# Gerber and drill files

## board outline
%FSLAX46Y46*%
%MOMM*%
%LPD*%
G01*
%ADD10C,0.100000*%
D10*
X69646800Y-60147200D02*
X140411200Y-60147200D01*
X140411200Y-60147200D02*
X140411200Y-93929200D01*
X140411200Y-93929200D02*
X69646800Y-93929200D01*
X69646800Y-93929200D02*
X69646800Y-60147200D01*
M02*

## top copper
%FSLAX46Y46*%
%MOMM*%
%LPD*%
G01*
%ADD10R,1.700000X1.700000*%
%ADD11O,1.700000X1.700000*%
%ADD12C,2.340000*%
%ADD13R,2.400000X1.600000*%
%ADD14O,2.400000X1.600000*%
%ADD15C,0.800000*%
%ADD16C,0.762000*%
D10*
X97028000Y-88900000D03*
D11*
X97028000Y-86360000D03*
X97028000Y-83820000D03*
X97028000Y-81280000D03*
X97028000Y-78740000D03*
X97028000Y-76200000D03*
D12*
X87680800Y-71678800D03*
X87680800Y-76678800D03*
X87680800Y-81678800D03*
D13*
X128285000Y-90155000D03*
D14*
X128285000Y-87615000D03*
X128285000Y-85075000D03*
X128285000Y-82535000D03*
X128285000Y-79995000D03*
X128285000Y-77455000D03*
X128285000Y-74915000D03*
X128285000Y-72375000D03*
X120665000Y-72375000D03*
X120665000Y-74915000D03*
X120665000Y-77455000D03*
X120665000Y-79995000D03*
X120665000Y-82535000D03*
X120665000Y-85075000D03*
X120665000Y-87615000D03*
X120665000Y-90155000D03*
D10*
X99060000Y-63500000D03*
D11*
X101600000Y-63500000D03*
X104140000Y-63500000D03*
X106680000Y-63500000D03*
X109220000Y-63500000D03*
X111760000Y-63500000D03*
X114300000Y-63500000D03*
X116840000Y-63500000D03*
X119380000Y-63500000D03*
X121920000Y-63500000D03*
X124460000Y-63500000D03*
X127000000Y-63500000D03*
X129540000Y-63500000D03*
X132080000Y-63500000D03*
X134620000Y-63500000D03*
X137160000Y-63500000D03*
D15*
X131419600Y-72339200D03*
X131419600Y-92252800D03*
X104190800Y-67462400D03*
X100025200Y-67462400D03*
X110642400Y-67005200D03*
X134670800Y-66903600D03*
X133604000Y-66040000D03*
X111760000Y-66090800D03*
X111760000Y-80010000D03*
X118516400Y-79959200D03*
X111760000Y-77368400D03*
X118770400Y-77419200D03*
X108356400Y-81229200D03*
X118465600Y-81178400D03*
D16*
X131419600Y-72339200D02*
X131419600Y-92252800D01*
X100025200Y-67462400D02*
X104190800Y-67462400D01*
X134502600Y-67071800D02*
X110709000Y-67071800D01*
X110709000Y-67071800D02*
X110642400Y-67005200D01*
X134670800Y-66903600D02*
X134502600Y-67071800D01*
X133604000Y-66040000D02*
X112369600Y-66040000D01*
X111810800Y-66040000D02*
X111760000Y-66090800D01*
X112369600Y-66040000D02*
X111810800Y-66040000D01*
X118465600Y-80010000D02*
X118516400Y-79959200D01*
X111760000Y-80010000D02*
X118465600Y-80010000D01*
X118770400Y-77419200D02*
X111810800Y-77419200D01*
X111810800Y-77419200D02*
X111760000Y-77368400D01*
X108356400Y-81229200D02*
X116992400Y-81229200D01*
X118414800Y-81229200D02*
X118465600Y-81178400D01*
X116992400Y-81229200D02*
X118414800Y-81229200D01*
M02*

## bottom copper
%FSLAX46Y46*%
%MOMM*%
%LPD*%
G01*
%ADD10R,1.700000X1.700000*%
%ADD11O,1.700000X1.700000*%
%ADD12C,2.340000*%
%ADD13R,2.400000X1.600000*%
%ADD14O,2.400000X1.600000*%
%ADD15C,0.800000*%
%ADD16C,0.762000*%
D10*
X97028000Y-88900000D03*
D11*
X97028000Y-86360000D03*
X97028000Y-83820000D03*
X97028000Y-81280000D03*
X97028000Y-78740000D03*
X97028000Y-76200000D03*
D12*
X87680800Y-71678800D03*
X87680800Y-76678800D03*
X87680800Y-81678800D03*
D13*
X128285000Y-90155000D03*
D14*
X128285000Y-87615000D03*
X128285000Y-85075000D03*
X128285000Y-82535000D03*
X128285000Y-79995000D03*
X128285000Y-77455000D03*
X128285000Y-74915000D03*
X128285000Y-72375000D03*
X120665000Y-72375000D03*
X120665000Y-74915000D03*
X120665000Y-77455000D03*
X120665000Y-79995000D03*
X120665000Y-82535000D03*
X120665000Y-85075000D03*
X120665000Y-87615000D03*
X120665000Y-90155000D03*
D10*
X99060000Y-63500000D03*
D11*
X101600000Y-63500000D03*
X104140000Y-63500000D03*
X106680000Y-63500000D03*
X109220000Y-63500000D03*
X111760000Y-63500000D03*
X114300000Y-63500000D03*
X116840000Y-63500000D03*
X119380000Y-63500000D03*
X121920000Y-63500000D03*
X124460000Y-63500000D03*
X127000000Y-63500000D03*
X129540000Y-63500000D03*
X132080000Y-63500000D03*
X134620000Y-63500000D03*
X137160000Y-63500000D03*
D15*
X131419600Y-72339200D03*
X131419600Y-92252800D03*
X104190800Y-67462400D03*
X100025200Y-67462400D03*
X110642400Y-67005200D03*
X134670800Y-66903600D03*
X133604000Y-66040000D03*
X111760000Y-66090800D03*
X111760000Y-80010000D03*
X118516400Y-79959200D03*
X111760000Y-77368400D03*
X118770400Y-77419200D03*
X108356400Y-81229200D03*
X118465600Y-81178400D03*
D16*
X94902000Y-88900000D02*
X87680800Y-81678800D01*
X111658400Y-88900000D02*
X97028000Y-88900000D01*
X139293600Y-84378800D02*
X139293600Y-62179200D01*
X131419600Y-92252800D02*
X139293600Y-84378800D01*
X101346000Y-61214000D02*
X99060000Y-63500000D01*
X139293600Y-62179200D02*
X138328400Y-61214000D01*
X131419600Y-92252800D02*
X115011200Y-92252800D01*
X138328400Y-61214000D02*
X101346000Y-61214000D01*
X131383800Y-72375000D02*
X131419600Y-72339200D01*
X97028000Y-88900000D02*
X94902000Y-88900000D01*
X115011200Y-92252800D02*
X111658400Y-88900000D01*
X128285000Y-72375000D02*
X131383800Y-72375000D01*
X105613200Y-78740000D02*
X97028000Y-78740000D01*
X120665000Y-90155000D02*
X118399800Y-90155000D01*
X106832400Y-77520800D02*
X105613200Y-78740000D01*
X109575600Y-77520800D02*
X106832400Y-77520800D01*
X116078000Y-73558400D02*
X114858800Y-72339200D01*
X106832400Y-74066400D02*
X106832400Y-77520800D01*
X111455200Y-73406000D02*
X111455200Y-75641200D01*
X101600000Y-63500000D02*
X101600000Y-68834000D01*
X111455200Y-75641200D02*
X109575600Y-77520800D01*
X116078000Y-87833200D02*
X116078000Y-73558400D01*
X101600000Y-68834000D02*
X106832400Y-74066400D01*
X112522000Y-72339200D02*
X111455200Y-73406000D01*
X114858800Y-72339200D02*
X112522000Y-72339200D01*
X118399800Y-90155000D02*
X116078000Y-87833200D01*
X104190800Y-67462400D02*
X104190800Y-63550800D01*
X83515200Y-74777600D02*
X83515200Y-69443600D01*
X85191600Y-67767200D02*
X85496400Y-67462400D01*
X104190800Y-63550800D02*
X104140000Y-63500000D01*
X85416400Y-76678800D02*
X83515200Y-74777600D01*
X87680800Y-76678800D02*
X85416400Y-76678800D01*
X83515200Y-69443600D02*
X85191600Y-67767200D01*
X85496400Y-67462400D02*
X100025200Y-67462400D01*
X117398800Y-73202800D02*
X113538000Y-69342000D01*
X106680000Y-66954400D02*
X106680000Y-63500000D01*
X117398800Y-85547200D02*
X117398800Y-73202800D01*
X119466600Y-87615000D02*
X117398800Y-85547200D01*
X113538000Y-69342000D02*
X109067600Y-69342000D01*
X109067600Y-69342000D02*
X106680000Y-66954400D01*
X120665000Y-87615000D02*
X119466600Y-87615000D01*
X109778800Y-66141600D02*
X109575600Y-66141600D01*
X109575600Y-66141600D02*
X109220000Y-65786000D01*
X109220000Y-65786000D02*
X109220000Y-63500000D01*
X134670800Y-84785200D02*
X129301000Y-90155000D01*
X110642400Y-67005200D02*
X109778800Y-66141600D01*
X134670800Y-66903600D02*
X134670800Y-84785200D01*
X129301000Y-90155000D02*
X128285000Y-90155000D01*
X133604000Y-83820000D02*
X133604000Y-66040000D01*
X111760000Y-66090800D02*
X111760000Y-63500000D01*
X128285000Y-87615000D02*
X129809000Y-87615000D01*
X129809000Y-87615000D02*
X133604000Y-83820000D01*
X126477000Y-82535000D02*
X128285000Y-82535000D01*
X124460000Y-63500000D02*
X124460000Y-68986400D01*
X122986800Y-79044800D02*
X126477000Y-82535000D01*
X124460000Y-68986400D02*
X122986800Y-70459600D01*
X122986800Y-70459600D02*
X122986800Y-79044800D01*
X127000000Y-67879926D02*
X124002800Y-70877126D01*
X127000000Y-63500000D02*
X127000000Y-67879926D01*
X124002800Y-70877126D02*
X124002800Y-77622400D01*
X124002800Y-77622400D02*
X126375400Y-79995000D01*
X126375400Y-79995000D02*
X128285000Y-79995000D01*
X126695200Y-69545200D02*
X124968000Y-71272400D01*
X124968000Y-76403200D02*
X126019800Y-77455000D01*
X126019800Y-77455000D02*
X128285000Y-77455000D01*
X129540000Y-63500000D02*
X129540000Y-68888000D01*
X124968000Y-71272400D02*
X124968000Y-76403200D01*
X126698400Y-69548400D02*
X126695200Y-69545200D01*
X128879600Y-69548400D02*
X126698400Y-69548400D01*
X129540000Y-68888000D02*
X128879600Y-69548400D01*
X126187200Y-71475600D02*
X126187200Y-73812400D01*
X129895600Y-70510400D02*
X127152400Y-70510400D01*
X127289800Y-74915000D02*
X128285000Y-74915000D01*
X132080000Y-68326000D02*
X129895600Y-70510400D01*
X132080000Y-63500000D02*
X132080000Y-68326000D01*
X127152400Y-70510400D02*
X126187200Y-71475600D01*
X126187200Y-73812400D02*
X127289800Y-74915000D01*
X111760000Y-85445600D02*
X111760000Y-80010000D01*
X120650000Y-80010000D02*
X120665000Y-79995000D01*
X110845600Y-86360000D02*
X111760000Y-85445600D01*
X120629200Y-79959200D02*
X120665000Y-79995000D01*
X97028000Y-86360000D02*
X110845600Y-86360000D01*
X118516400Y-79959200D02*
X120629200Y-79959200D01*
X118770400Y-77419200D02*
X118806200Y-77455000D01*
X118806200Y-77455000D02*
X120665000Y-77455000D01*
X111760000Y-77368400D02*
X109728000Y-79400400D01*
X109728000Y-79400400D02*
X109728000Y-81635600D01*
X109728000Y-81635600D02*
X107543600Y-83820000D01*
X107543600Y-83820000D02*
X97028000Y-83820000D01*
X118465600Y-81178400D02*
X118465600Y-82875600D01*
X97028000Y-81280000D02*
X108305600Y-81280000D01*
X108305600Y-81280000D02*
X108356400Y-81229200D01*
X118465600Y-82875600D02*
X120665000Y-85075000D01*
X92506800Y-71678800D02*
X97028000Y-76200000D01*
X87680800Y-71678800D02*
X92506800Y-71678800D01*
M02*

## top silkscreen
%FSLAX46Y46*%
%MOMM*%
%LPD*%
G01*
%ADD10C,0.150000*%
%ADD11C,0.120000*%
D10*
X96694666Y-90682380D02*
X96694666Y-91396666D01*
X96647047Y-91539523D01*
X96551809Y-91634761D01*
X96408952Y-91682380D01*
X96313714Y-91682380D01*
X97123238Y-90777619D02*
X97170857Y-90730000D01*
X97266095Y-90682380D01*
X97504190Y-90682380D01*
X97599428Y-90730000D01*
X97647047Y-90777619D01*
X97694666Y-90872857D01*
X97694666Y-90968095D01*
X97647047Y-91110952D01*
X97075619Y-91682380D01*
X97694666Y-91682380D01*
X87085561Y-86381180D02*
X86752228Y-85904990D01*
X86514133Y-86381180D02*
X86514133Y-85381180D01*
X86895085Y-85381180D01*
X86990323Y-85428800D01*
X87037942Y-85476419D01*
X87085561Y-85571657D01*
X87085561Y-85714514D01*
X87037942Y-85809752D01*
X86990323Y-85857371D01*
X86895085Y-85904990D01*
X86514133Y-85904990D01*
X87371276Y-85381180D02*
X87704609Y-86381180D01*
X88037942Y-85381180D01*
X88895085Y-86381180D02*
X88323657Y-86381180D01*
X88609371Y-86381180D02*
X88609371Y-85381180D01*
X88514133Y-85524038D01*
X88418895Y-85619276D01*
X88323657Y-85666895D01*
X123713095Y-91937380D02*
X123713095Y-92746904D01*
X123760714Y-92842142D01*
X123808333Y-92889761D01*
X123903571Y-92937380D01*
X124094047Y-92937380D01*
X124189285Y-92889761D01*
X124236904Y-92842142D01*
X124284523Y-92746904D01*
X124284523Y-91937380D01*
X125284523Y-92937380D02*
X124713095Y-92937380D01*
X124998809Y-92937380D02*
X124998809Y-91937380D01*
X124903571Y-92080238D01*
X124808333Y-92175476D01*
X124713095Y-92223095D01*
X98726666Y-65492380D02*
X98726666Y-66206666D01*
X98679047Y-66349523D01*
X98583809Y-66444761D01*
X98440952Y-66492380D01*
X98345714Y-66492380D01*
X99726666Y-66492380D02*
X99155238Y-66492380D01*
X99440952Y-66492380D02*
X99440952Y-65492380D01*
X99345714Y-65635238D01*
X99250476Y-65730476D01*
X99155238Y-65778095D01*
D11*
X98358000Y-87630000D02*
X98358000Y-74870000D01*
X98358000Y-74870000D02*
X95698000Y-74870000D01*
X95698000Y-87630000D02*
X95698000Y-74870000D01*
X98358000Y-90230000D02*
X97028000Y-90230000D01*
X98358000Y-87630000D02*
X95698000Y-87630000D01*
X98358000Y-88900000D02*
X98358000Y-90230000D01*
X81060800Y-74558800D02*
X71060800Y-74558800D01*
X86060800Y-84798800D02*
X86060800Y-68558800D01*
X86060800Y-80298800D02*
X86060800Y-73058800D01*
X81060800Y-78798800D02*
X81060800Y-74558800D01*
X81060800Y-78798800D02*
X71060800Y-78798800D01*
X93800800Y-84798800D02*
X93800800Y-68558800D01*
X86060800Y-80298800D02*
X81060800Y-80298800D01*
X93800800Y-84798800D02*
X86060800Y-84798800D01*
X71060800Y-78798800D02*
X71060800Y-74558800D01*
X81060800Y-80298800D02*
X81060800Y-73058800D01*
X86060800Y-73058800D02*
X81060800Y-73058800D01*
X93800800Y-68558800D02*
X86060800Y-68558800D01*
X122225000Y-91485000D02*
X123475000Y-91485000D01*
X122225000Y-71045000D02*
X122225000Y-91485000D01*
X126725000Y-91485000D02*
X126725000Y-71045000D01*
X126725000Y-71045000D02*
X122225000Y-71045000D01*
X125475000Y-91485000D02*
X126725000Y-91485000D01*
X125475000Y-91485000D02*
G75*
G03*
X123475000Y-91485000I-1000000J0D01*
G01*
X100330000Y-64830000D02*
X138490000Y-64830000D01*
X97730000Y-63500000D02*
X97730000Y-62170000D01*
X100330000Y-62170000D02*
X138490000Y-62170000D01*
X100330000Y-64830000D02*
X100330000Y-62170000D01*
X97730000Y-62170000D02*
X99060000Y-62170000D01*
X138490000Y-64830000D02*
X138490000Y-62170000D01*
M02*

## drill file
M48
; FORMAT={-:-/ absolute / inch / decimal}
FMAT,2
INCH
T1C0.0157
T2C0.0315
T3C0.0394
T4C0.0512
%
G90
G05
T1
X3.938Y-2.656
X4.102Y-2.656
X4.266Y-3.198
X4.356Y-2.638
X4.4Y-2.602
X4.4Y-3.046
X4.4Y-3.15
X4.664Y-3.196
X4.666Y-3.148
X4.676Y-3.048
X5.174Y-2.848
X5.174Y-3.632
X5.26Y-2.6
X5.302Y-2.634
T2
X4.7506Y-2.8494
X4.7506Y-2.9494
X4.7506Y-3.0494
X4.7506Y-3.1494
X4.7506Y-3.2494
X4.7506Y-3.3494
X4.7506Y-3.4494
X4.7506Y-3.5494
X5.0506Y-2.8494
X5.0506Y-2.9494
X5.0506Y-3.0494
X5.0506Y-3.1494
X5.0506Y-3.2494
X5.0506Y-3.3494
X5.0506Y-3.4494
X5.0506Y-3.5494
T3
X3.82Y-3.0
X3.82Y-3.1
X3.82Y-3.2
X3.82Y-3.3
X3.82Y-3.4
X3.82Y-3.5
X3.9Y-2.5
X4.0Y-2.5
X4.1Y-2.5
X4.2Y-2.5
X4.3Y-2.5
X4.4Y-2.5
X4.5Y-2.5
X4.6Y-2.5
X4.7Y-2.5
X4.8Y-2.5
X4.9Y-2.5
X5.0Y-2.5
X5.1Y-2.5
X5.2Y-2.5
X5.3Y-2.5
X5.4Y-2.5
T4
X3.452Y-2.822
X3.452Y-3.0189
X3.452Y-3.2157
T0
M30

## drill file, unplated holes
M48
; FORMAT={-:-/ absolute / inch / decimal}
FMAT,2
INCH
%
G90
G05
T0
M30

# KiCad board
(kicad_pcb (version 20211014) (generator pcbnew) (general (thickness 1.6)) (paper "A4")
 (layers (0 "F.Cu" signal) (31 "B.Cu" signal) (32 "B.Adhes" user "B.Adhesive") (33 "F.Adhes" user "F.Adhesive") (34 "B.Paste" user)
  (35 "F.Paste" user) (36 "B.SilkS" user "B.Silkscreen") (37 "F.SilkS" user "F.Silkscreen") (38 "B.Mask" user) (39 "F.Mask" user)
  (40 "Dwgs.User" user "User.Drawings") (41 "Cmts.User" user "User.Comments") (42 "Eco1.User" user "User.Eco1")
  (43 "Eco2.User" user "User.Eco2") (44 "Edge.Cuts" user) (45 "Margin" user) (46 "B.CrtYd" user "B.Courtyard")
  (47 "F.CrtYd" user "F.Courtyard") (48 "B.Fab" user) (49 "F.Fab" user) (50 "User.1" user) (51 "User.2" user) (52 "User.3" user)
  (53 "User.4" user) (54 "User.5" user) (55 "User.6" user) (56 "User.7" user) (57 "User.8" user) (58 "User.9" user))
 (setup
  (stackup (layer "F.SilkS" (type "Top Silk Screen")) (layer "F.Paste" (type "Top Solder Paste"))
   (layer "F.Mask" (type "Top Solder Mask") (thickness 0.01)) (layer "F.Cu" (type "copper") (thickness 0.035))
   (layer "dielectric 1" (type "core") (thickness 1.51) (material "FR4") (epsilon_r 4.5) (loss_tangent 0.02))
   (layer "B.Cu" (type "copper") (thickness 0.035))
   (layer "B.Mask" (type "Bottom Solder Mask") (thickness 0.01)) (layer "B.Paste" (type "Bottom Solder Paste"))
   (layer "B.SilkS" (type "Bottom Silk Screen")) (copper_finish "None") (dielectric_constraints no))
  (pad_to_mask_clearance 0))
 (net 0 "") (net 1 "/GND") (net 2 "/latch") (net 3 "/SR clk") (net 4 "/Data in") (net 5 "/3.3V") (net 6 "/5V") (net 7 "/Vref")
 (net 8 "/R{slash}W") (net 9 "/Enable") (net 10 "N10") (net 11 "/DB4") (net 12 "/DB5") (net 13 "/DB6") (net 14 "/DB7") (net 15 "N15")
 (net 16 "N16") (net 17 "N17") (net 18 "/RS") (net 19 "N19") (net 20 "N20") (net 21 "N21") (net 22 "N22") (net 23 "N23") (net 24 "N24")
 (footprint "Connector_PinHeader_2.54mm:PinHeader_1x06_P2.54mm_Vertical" (layer "F.Cu") (at 97.028 88.9 180)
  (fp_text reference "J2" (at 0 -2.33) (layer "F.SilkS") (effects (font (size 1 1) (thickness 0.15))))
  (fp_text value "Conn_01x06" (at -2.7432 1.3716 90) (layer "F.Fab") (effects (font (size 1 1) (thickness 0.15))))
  (fp_line (start -1.33 1.27) (end -1.33 14.03) (layer "F.SilkS") (width 0.12))
  (fp_line (start -1.33 14.03) (end 1.33 14.03) (layer "F.SilkS") (width 0.12))
  (fp_line (start 1.33 1.27) (end 1.33 14.03) (layer "F.SilkS") (width 0.12))
  (fp_line (start -1.33 -1.33) (end 0 -1.33) (layer "F.SilkS") (width 0.12))
  (fp_line (start -1.33 1.27) (end 1.33 1.27) (layer "F.SilkS") (width 0.12))
  (fp_line (start -1.33 0) (end -1.33 -1.33) (layer "F.SilkS") (width 0.12))
  (pad "1" thru_hole rect (at 0 0 180) (size 1.7 1.7) (drill 1) (layers *.Cu *.Mask) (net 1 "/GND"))
  (pad "2" thru_hole oval (at 0 2.54 180) (size 1.7 1.7) (drill 1) (layers *.Cu *.Mask) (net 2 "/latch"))
  (pad "3" thru_hole oval (at 0 5.08 180) (size 1.7 1.7) (drill 1) (layers *.Cu *.Mask) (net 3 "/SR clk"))
  (pad "4" thru_hole oval (at 0 7.62 180) (size 1.7 1.7) (drill 1) (layers *.Cu *.Mask) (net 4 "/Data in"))
  (pad "5" thru_hole oval (at 0 10.16 180) (size 1.7 1.7) (drill 1) (layers *.Cu *.Mask) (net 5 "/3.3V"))
  (pad "6" thru_hole oval (at 0 12.7 180) (size 1.7 1.7) (drill 1) (layers *.Cu *.Mask) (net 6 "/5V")))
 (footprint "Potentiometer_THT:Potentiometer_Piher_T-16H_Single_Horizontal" (layer "F.Cu") (at 87.6808 71.6788 180)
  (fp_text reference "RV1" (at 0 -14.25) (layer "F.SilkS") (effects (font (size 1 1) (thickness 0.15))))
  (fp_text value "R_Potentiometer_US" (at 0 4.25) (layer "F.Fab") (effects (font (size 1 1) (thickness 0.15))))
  (fp_line (start 6.62 -2.88) (end 16.62 -2.88) (layer "F.SilkS") (width 0.12))
  (fp_line (start 1.62 -13.12) (end 1.62 3.12) (layer "F.SilkS") (width 0.12))
  (fp_line (start 1.62 -8.62) (end 1.62 -1.38) (layer "F.SilkS") (width 0.12))
  (fp_line (start 6.62 -7.12) (end 6.62 -2.88) (layer "F.SilkS") (width 0.12))
  (fp_line (start 6.62 -7.12) (end 16.62 -7.12) (layer "F.SilkS") (width 0.12))
  (fp_line (start -6.12 -13.12) (end -6.12 3.12) (layer "F.SilkS") (width 0.12))
  (fp_line (start 1.62 -8.62) (end 6.62 -8.62) (layer "F.SilkS") (width 0.12))
  (fp_line (start -6.12 -13.12) (end 1.62 -13.12) (layer "F.SilkS") (width 0.12))
  (fp_line (start 16.62 -7.12) (end 16.62 -2.88) (layer "F.SilkS") (width 0.12))
  (fp_line (start 6.62 -8.62) (end 6.62 -1.38) (layer "F.SilkS") (width 0.12))
  (fp_line (start 1.62 -1.38) (end 6.62 -1.38) (layer "F.SilkS") (width 0.12))
  (fp_line (start -6.12 3.12) (end 1.62 3.12) (layer "F.SilkS") (width 0.12))
  (pad "1" thru_hole circle (at 0 0 180) (size 2.34 2.34) (drill 1.3) (layers *.Cu *.Mask) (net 6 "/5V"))
  (pad "2" thru_hole circle (at 0 -5 180) (size 2.34 2.34) (drill 1.3) (layers *.Cu *.Mask) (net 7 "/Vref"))
  (pad "3" thru_hole circle (at 0 -10 180) (size 2.34 2.34) (drill 1.3) (layers *.Cu *.Mask) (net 1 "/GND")))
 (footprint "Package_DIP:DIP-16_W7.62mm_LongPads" (layer "F.Cu") (at 128.285 90.155 180)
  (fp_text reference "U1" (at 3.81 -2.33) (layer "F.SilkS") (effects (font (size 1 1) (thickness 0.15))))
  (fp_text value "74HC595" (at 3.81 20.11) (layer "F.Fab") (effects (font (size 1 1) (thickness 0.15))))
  (fp_line (start 6.06 -1.33) (end 4.81 -1.33) (layer "F.SilkS") (width 0.12))
  (fp_line (start 6.06 19.11) (end 6.06 -1.33) (layer "F.SilkS") (width 0.12))
  (fp_line (start 1.56 -1.33) (end 1.56 19.11) (layer "F.SilkS") (width 0.12))
  (fp_line (start 1.56 19.11) (end 6.06 19.11) (layer "F.SilkS") (width 0.12))
  (fp_line (start 2.81 -1.33) (end 1.56 -1.33) (layer "F.SilkS") (width 0.12))
  (fp_arc (start 4.81 -1.33) (mid 3.81 -0.33) (end 2.81 -1.33) (layer "F.SilkS") (width 0.12))
  (pad "1" thru_hole rect (at 0 0 180) (size 2.4 1.6) (drill 0.8) (layers *.Cu *.Mask) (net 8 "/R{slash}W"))
  (pad "2" thru_hole oval (at 0 2.54 180) (size 2.4 1.6) (drill 0.8) (layers *.Cu *.Mask) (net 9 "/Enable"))
  (pad "3" thru_hole oval (at 0 5.08 180) (size 2.4 1.6) (drill 0.8) (layers *.Cu *.Mask) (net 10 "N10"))
  (pad "4" thru_hole oval (at 0 7.62 180) (size 2.4 1.6) (drill 0.8) (layers *.Cu *.Mask) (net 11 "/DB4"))
  (pad "5" thru_hole oval (at 0 10.16 180) (size 2.4 1.6) (drill 0.8) (layers *.Cu *.Mask) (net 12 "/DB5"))
  (pad "6" thru_hole oval (at 0 12.7 180) (size 2.4 1.6) (drill 0.8) (layers *.Cu *.Mask) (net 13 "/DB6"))
  (pad "7" thru_hole oval (at 0 15.24 180) (size 2.4 1.6) (drill 0.8) (layers *.Cu *.Mask) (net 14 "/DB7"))
  (pad "8" thru_hole oval (at 0 17.78 180) (size 2.4 1.6) (drill 0.8) (layers *.Cu *.Mask) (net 1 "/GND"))
  (pad "9" thru_hole oval (at 7.62 17.78 180) (size 2.4 1.6) (drill 0.8) (layers *.Cu *.Mask) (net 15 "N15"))
  (pad "10" thru_hole oval (at 7.62 15.24 180) (size 2.4 1.6) (drill 0.8) (layers *.Cu *.Mask) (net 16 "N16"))
  (pad "11" thru_hole oval (at 7.62 12.7 180) (size 2.4 1.6) (drill 0.8) (layers *.Cu *.Mask) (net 3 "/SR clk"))
  (pad "12" thru_hole oval (at 7.62 10.16 180) (size 2.4 1.6) (drill 0.8) (layers *.Cu *.Mask) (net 2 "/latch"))
  (pad "13" thru_hole oval (at 7.62 7.62 180) (size 2.4 1.6) (drill 0.8) (layers *.Cu *.Mask) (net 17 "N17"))
  (pad "14" thru_hole oval (at 7.62 5.08 180) (size 2.4 1.6) (drill 0.8) (layers *.Cu *.Mask) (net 4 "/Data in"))
  (pad "15" thru_hole oval (at 7.62 2.54 180) (size 2.4 1.6) (drill 0.8) (layers *.Cu *.Mask) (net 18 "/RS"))
  (pad "16" thru_hole oval (at 7.62 0 180) (size 2.4 1.6) (drill 0.8) (layers *.Cu *.Mask) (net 5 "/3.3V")))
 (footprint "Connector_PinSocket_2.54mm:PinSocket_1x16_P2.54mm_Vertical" (layer "F.Cu") (at 99.06 63.5 90)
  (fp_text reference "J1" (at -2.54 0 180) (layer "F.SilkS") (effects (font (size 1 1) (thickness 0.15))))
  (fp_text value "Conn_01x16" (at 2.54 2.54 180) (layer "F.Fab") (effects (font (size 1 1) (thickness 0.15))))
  (fp_line (start -1.33 1.27) (end -1.33 39.43) (layer "F.SilkS") (width 0.12))
  (fp_line (start 0 -1.33) (end 1.33 -1.33) (layer "F.SilkS") (width 0.12))
  (fp_line (start 1.33 1.27) (end 1.33 39.43) (layer "F.SilkS") (width 0.12))
  (fp_line (start -1.33 1.27) (end 1.33 1.27) (layer "F.SilkS") (width 0.12))
  (fp_line (start 1.33 -1.33) (end 1.33 0) (layer "F.SilkS") (width 0.12))
  (fp_line (start -1.33 39.43) (end 1.33 39.43) (layer "F.SilkS") (width 0.12))
  (pad "1" thru_hole rect (at 0 0 90) (size 1.7 1.7) (drill 1) (layers *.Cu *.Mask) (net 1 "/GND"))
  (pad "2" thru_hole oval (at 0 2.54 90) (size 1.7 1.7) (drill 1) (layers *.Cu *.Mask) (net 5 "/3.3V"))
  (pad "3" thru_hole oval (at 0 5.08 90) (size 1.7 1.7) (drill 1) (layers *.Cu *.Mask) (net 7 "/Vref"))
  (pad "4" thru_hole oval (at 0 7.62 90) (size 1.7 1.7) (drill 1) (layers *.Cu *.Mask) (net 18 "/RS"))
  (pad "5" thru_hole oval (at 0 10.16 90) (size 1.7 1.7) (drill 1) (layers *.Cu *.Mask) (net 8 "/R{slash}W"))
  (pad "6" thru_hole oval (at 0 12.7 90) (size 1.7 1.7) (drill 1) (layers *.Cu *.Mask) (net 9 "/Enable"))
  (pad "7" thru_hole oval (at 0 15.24 90) (size 1.7 1.7) (drill 1) (layers *.Cu *.Mask) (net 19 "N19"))
  (pad "8" thru_hole oval (at 0 17.78 90) (size 1.7 1.7) (drill 1) (layers *.Cu *.Mask) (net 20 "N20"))
  (pad "9" thru_hole oval (at 0 20.32 90) (size 1.7 1.7) (drill 1) (layers *.Cu *.Mask) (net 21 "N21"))
  (pad "10" thru_hole oval (at 0 22.86 90) (size 1.7 1.7) (drill 1) (layers *.Cu *.Mask) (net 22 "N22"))
  (pad "11" thru_hole oval (at 0 25.4 90) (size 1.7 1.7) (drill 1) (layers *.Cu *.Mask) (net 11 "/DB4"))
  (pad "12" thru_hole oval (at 0 27.94 90) (size 1.7 1.7) (drill 1) (layers *.Cu *.Mask) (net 12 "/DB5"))
  (pad "13" thru_hole oval (at 0 30.48 90) (size 1.7 1.7) (drill 1) (layers *.Cu *.Mask) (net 13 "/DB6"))
  (pad "14" thru_hole oval (at 0 33.02 90) (size 1.7 1.7) (drill 1) (layers *.Cu *.Mask) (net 14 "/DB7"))
  (pad "15" thru_hole oval (at 0 35.56 90) (size 1.7 1.7) (drill 1) (layers *.Cu *.Mask) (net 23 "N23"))
  (pad "16" thru_hole oval (at 0 38.1 90) (size 1.7 1.7) (drill 1) (layers *.Cu *.Mask) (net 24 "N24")))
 (gr_rect (start 69.6468 60.1472) (end 140.4112 93.9292) (layer "Edge.Cuts") (width 0.1) (fill none))
 (segment (start 131.4196 72.3392) (end 131.4196 92.2528) (width 0.762) (layer "F.Cu") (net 1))
 (via (at 131.4196 72.3392) (size 0.8) (drill 0.4) (layers "F.Cu" "B.Cu") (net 1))
 (via (at 131.4196 92.2528) (size 0.8) (drill 0.4) (layers "F.Cu" "B.Cu") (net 1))
 (segment (start 94.902 88.9) (end 87.6808 81.6788) (width 0.762) (layer "B.Cu") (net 1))
 (segment (start 111.6584 88.9) (end 97.028 88.9) (width 0.762) (layer "B.Cu") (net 1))
 (segment (start 139.2936 84.3788) (end 139.2936 62.1792) (width 0.762) (layer "B.Cu") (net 1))
 (segment (start 131.4196 92.2528) (end 139.2936 84.3788) (width 0.762) (layer "B.Cu") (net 1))
 (segment (start 101.346 61.214) (end 99.06 63.5) (width 0.762) (layer "B.Cu") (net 1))
 (segment (start 139.2936 62.1792) (end 138.3284 61.214) (width 0.762) (layer "B.Cu") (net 1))
 (segment (start 131.4196 92.2528) (end 115.0112 92.2528) (width 0.762) (layer "B.Cu") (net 1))
 (segment (start 138.3284 61.214) (end 101.346 61.214) (width 0.762) (layer "B.Cu") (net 1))
 (segment (start 131.3838 72.375) (end 131.4196 72.3392) (width 0.762) (layer "B.Cu") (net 1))
 (segment (start 97.028 88.9) (end 94.902 88.9) (width 0.762) (layer "B.Cu") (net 1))
 (segment (start 115.0112 92.2528) (end 111.6584 88.9) (width 0.762) (layer "B.Cu") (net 1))
 (segment (start 128.285 72.375) (end 131.3838 72.375) (width 0.762) (layer "B.Cu") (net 1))
 (segment (start 105.6132 78.74) (end 97.028 78.74) (width 0.762) (layer "B.Cu") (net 5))
 (segment (start 120.665 90.155) (end 118.3998 90.155) (width 0.762) (layer "B.Cu") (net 5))
 (segment (start 106.8324 77.5208) (end 105.6132 78.74) (width 0.762) (layer "B.Cu") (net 5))
 (segment (start 109.5756 77.5208) (end 106.8324 77.5208) (width 0.762) (layer "B.Cu") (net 5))
 (segment (start 116.078 73.5584) (end 114.8588 72.3392) (width 0.762) (layer "B.Cu") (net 5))
 (segment (start 106.8324 74.0664) (end 106.8324 77.5208) (width 0.762) (layer "B.Cu") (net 5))
 (segment (start 111.4552 73.406) (end 111.4552 75.6412) (width 0.762) (layer "B.Cu") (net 5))
 (segment (start 101.6 63.5) (end 101.6 68.834) (width 0.762) (layer "B.Cu") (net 5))
 (segment (start 111.4552 75.6412) (end 109.5756 77.5208) (width 0.762) (layer "B.Cu") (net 5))
 (segment (start 116.078 87.8332) (end 116.078 73.5584) (width 0.762) (layer "B.Cu") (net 5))
 (segment (start 101.6 68.834) (end 106.8324 74.0664) (width 0.762) (layer "B.Cu") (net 5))
 (segment (start 112.522 72.3392) (end 111.4552 73.406) (width 0.762) (layer "B.Cu") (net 5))
 (segment (start 114.8588 72.3392) (end 112.522 72.3392) (width 0.762) (layer "B.Cu") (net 5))
 (segment (start 118.3998 90.155) (end 116.078 87.8332) (width 0.762) (layer "B.Cu") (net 5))
 (segment (start 100.0252 67.4624) (end 104.1908 67.4624) (width 0.762) (layer "F.Cu") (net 7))
 (via (at 104.1908 67.4624) (size 0.8) (drill 0.4) (layers "F.Cu" "B.Cu") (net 7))
 (via (at 100.0252 67.4624) (size 0.8) (drill 0.4) (layers "F.Cu" "B.Cu") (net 7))
 (segment (start 104.1908 67.4624) (end 104.1908 63.5508) (width 0.762) (layer "B.Cu") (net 7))
 (segment (start 83.5152 74.7776) (end 83.5152 69.4436) (width 0.762) (layer "B.Cu") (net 7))
 (segment (start 85.1916 67.7672) (end 85.4964 67.4624) (width 0.762) (layer "B.Cu") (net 7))
 (segment (start 104.1908 63.5508) (end 104.14 63.5) (width 0.762) (layer "B.Cu") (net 7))
 (segment (start 85.4164 76.6788) (end 83.5152 74.7776) (width 0.762) (layer "B.Cu") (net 7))
 (segment (start 87.6808 76.6788) (end 85.4164 76.6788) (width 0.762) (layer "B.Cu") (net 7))
 (segment (start 83.5152 69.4436) (end 85.1916 67.7672) (width 0.762) (layer "B.Cu") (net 7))
 (segment (start 85.4964 67.4624) (end 100.0252 67.4624) (width 0.762) (layer "B.Cu") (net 7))
 (segment (start 117.3988 73.2028) (end 113.538 69.342) (width 0.762) (layer "B.Cu") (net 18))
 (segment (start 106.68 66.9544) (end 106.68 63.5) (width 0.762) (layer "B.Cu") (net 18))
 (segment (start 117.3988 85.5472) (end 117.3988 73.2028) (width 0.762) (layer "B.Cu") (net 18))
 (segment (start 119.4666 87.615) (end 117.3988 85.5472) (width 0.762) (layer "B.Cu") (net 18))
 (segment (start 113.538 69.342) (end 109.0676 69.342) (width 0.762) (layer "B.Cu") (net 18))
 (segment (start 109.0676 69.342) (end 106.68 66.9544) (width 0.762) (layer "B.Cu") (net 18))
 (segment (start 120.665 87.615) (end 119.4666 87.615) (width 0.762) (layer "B.Cu") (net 18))
 (segment (start 134.5026 67.0718) (end 110.709 67.0718) (width 0.762) (layer "F.Cu") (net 8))
 (segment (start 110.709 67.0718) (end 110.6424 67.0052) (width 0.762) (layer "F.Cu") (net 8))
 (segment (start 134.6708 66.9036) (end 134.5026 67.0718) (width 0.762) (layer "F.Cu") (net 8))
 (via (at 110.6424 67.0052) (size 0.8) (drill 0.4) (layers "F.Cu" "B.Cu") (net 8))
 (via (at 134.6708 66.9036) (size 0.8) (drill 0.4) (layers "F.Cu" "B.Cu") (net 8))
 (segment (start 109.7788 66.1416) (end 109.5756 66.1416) (width 0.762) (layer "B.Cu") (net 8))
 (segment (start 109.5756 66.1416) (end 109.22 65.786) (width 0.762) (layer "B.Cu") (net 8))
 (segment (start 109.22 65.786) (end 109.22 63.5) (width 0.762) (layer "B.Cu") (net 8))
 (segment (start 134.6708 84.7852) (end 129.301 90.155) (width 0.762) (layer "B.Cu") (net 8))
 (segment (start 110.6424 67.0052) (end 109.7788 66.1416) (width 0.762) (layer "B.Cu") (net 8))
 (segment (start 134.6708 66.9036) (end 134.6708 84.7852) (width 0.762) (layer "B.Cu") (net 8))
 (segment (start 129.301 90.155) (end 128.285 90.155) (width 0.762) (layer "B.Cu") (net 8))
 (segment (start 133.604 66.04) (end 112.3696 66.04) (width 0.762) (layer "F.Cu") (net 9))
 (segment (start 111.8108 66.04) (end 111.76 66.0908) (width 0.762) (layer "F.Cu") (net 9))
 (segment (start 112.3696 66.04) (end 111.8108 66.04) (width 0.762) (layer "F.Cu") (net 9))
 (via (at 133.604 66.04) (size 0.8) (drill 0.4) (layers "F.Cu" "B.Cu") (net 9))
 (via (at 111.76 66.0908) (size 0.8) (drill 0.4) (layers "F.Cu" "B.Cu") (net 9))
 (segment (start 133.604 83.82) (end 133.604 66.04) (width 0.762) (layer "B.Cu") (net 9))
 (segment (start 111.76 66.0908) (end 111.76 63.5) (width 0.762) (layer "B.Cu") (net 9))
 (segment (start 128.285 87.615) (end 129.809 87.615) (width 0.762) (layer "B.Cu") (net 9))
 (segment (start 129.809 87.615) (end 133.604 83.82) (width 0.762) (layer "B.Cu") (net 9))
 (segment (start 126.477 82.535) (end 128.285 82.535) (width 0.762) (layer "B.Cu") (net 11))
 (segment (start 124.46 63.5) (end 124.46 68.9864) (width 0.762) (layer "B.Cu") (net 11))
 (segment (start 122.9868 79.0448) (end 126.477 82.535) (width 0.762) (layer "B.Cu") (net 11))
 (segment (start 124.46 68.9864) (end 122.9868 70.4596) (width 0.762) (layer "B.Cu") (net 11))
 (segment (start 122.9868 70.4596) (end 122.9868 79.0448) (width 0.762) (layer "B.Cu") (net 11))
 (segment (start 127 67.879926) (end 124.0028 70.877126) (width 0.762) (layer "B.Cu") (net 12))
 (segment (start 127 63.5) (end 127 67.879926) (width 0.762) (layer "B.Cu") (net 12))
 (segment (start 124.0028 70.877126) (end 124.0028 77.6224) (width 0.762) (layer "B.Cu") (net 12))
 (segment (start 124.0028 77.6224) (end 126.3754 79.995) (width 0.762) (layer "B.Cu") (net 12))
 (segment (start 126.3754 79.995) (end 128.285 79.995) (width 0.762) (layer "B.Cu") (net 12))
 (segment (start 126.6952 69.5452) (end 124.968 71.2724) (width 0.762) (layer "B.Cu") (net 13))
 (segment (start 124.968 76.4032) (end 126.0198 77.455) (width 0.762) (layer "B.Cu") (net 13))
 (segment (start 126.0198 77.455) (end 128.285 77.455) (width 0.762) (layer "B.Cu") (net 13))
 (segment (start 129.54 63.5) (end 129.54 68.888) (width 0.762) (layer "B.Cu") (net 13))
 (segment (start 124.968 71.2724) (end 124.968 76.4032) (width 0.762) (layer "B.Cu") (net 13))
 (segment (start 126.6984 69.5484) (end 126.6952 69.5452) (width 0.762) (layer "B.Cu") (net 13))
 (segment (start 128.8796 69.5484) (end 126.6984 69.5484) (width 0.762) (layer "B.Cu") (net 13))
 (segment (start 129.54 68.888) (end 128.8796 69.5484) (width 0.762) (layer "B.Cu") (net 13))
 (segment (start 126.1872 71.4756) (end 126.1872 73.8124) (width 0.762) (layer "B.Cu") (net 14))
 (segment (start 129.8956 70.5104) (end 127.1524 70.5104) (width 0.762) (layer "B.Cu") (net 14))
 (segment (start 127.2898 74.915) (end 128.285 74.915) (width 0.762) (layer "B.Cu") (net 14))
 (segment (start 132.08 68.326) (end 129.8956 70.5104) (width 0.762) (layer "B.Cu") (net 14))
 (segment (start 132.08 63.5) (end 132.08 68.326) (width 0.762) (layer "B.Cu") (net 14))
 (segment (start 127.1524 70.5104) (end 126.1872 71.4756) (width 0.762) (layer "B.Cu") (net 14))
 (segment (start 126.1872 73.8124) (end 127.2898 74.915) (width 0.762) (layer "B.Cu") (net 14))
 (segment (start 118.4656 80.01) (end 118.5164 79.9592) (width 0.762) (layer "F.Cu") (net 2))
 (segment (start 111.76 80.01) (end 118.4656 80.01) (width 0.762) (layer "F.Cu") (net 2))
 (via (at 111.76 80.01) (size 0.8) (drill 0.4) (layers "F.Cu" "B.Cu") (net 2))
 (via (at 118.5164 79.9592) (size 0.8) (drill 0.4) (layers "F.Cu" "B.Cu") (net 2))
 (segment (start 111.76 85.4456) (end 111.76 80.01) (width 0.762) (layer "B.Cu") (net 2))
 (segment (start 120.65 80.01) (end 120.665 79.995) (width 0.762) (layer "B.Cu") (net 2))
 (segment (start 110.8456 86.36) (end 111.76 85.4456) (width 0.762) (layer "B.Cu") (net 2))
 (segment (start 120.6292 79.9592) (end 120.665 79.995) (width 0.762) (layer "B.Cu") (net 2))
 (segment (start 97.028 86.36) (end 110.8456 86.36) (width 0.762) (layer "B.Cu") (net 2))
 (segment (start 118.5164 79.9592) (end 120.6292 79.9592) (width 0.762) (layer "B.Cu") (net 2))
 (segment (start 118.7704 77.4192) (end 111.8108 77.4192) (width 0.762) (layer "F.Cu") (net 3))
 (segment (start 111.8108 77.4192) (end 111.76 77.3684) (width 0.762) (layer "F.Cu") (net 3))
 (via (at 111.76 77.3684) (size 0.8) (drill 0.4) (layers "F.Cu" "B.Cu") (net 3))
 (via (at 118.7704 77.4192) (size 0.8) (drill 0.4) (layers "F.Cu" "B.Cu") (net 3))
 (segment (start 118.7704 77.4192) (end 118.8062 77.455) (width 0.762) (layer "B.Cu") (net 3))
 (segment (start 118.8062 77.455) (end 120.665 77.455) (width 0.762) (layer "B.Cu") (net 3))
 (segment (start 111.76 77.3684) (end 109.728 79.4004) (width 0.762) (layer "B.Cu") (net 3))
 (segment (start 109.728 79.4004) (end 109.728 81.6356) (width 0.762) (layer "B.Cu") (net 3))
 (segment (start 109.728 81.6356) (end 107.5436 83.82) (width 0.762) (layer "B.Cu") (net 3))
 (segment (start 107.5436 83.82) (end 97.028 83.82) (width 0.762) (layer "B.Cu") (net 3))
 (segment (start 108.3564 81.2292) (end 116.9924 81.2292) (width 0.762) (layer "F.Cu") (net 4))
 (segment (start 118.4148 81.2292) (end 118.4656 81.1784) (width 0.762) (layer "F.Cu") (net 4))
 (segment (start 116.9924 81.2292) (end 118.4148 81.2292) (width 0.762) (layer "F.Cu") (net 4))
 (via (at 108.3564 81.2292) (size 0.8) (drill 0.4) (layers "F.Cu" "B.Cu") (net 4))
 (via (at 118.4656 81.1784) (size 0.8) (drill 0.4) (layers "F.Cu" "B.Cu") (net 4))
 (segment (start 118.4656 81.1784) (end 118.4656 82.8756) (width 0.762) (layer "B.Cu") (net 4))
 (segment (start 97.028 81.28) (end 108.3056 81.28) (width 0.762) (layer "B.Cu") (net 4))
 (segment (start 108.3056 81.28) (end 108.3564 81.2292) (width 0.762) (layer "B.Cu") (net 4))
 (segment (start 118.4656 82.8756) (end 120.665 85.075) (width 0.762) (layer "B.Cu") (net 4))
 (segment (start 92.5068 71.6788) (end 97.028 76.2) (width 0.762) (layer "B.Cu") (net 6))
 (segment (start 87.6808 71.6788) (end 92.5068 71.6788) (width 0.762) (layer "B.Cu") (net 6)))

